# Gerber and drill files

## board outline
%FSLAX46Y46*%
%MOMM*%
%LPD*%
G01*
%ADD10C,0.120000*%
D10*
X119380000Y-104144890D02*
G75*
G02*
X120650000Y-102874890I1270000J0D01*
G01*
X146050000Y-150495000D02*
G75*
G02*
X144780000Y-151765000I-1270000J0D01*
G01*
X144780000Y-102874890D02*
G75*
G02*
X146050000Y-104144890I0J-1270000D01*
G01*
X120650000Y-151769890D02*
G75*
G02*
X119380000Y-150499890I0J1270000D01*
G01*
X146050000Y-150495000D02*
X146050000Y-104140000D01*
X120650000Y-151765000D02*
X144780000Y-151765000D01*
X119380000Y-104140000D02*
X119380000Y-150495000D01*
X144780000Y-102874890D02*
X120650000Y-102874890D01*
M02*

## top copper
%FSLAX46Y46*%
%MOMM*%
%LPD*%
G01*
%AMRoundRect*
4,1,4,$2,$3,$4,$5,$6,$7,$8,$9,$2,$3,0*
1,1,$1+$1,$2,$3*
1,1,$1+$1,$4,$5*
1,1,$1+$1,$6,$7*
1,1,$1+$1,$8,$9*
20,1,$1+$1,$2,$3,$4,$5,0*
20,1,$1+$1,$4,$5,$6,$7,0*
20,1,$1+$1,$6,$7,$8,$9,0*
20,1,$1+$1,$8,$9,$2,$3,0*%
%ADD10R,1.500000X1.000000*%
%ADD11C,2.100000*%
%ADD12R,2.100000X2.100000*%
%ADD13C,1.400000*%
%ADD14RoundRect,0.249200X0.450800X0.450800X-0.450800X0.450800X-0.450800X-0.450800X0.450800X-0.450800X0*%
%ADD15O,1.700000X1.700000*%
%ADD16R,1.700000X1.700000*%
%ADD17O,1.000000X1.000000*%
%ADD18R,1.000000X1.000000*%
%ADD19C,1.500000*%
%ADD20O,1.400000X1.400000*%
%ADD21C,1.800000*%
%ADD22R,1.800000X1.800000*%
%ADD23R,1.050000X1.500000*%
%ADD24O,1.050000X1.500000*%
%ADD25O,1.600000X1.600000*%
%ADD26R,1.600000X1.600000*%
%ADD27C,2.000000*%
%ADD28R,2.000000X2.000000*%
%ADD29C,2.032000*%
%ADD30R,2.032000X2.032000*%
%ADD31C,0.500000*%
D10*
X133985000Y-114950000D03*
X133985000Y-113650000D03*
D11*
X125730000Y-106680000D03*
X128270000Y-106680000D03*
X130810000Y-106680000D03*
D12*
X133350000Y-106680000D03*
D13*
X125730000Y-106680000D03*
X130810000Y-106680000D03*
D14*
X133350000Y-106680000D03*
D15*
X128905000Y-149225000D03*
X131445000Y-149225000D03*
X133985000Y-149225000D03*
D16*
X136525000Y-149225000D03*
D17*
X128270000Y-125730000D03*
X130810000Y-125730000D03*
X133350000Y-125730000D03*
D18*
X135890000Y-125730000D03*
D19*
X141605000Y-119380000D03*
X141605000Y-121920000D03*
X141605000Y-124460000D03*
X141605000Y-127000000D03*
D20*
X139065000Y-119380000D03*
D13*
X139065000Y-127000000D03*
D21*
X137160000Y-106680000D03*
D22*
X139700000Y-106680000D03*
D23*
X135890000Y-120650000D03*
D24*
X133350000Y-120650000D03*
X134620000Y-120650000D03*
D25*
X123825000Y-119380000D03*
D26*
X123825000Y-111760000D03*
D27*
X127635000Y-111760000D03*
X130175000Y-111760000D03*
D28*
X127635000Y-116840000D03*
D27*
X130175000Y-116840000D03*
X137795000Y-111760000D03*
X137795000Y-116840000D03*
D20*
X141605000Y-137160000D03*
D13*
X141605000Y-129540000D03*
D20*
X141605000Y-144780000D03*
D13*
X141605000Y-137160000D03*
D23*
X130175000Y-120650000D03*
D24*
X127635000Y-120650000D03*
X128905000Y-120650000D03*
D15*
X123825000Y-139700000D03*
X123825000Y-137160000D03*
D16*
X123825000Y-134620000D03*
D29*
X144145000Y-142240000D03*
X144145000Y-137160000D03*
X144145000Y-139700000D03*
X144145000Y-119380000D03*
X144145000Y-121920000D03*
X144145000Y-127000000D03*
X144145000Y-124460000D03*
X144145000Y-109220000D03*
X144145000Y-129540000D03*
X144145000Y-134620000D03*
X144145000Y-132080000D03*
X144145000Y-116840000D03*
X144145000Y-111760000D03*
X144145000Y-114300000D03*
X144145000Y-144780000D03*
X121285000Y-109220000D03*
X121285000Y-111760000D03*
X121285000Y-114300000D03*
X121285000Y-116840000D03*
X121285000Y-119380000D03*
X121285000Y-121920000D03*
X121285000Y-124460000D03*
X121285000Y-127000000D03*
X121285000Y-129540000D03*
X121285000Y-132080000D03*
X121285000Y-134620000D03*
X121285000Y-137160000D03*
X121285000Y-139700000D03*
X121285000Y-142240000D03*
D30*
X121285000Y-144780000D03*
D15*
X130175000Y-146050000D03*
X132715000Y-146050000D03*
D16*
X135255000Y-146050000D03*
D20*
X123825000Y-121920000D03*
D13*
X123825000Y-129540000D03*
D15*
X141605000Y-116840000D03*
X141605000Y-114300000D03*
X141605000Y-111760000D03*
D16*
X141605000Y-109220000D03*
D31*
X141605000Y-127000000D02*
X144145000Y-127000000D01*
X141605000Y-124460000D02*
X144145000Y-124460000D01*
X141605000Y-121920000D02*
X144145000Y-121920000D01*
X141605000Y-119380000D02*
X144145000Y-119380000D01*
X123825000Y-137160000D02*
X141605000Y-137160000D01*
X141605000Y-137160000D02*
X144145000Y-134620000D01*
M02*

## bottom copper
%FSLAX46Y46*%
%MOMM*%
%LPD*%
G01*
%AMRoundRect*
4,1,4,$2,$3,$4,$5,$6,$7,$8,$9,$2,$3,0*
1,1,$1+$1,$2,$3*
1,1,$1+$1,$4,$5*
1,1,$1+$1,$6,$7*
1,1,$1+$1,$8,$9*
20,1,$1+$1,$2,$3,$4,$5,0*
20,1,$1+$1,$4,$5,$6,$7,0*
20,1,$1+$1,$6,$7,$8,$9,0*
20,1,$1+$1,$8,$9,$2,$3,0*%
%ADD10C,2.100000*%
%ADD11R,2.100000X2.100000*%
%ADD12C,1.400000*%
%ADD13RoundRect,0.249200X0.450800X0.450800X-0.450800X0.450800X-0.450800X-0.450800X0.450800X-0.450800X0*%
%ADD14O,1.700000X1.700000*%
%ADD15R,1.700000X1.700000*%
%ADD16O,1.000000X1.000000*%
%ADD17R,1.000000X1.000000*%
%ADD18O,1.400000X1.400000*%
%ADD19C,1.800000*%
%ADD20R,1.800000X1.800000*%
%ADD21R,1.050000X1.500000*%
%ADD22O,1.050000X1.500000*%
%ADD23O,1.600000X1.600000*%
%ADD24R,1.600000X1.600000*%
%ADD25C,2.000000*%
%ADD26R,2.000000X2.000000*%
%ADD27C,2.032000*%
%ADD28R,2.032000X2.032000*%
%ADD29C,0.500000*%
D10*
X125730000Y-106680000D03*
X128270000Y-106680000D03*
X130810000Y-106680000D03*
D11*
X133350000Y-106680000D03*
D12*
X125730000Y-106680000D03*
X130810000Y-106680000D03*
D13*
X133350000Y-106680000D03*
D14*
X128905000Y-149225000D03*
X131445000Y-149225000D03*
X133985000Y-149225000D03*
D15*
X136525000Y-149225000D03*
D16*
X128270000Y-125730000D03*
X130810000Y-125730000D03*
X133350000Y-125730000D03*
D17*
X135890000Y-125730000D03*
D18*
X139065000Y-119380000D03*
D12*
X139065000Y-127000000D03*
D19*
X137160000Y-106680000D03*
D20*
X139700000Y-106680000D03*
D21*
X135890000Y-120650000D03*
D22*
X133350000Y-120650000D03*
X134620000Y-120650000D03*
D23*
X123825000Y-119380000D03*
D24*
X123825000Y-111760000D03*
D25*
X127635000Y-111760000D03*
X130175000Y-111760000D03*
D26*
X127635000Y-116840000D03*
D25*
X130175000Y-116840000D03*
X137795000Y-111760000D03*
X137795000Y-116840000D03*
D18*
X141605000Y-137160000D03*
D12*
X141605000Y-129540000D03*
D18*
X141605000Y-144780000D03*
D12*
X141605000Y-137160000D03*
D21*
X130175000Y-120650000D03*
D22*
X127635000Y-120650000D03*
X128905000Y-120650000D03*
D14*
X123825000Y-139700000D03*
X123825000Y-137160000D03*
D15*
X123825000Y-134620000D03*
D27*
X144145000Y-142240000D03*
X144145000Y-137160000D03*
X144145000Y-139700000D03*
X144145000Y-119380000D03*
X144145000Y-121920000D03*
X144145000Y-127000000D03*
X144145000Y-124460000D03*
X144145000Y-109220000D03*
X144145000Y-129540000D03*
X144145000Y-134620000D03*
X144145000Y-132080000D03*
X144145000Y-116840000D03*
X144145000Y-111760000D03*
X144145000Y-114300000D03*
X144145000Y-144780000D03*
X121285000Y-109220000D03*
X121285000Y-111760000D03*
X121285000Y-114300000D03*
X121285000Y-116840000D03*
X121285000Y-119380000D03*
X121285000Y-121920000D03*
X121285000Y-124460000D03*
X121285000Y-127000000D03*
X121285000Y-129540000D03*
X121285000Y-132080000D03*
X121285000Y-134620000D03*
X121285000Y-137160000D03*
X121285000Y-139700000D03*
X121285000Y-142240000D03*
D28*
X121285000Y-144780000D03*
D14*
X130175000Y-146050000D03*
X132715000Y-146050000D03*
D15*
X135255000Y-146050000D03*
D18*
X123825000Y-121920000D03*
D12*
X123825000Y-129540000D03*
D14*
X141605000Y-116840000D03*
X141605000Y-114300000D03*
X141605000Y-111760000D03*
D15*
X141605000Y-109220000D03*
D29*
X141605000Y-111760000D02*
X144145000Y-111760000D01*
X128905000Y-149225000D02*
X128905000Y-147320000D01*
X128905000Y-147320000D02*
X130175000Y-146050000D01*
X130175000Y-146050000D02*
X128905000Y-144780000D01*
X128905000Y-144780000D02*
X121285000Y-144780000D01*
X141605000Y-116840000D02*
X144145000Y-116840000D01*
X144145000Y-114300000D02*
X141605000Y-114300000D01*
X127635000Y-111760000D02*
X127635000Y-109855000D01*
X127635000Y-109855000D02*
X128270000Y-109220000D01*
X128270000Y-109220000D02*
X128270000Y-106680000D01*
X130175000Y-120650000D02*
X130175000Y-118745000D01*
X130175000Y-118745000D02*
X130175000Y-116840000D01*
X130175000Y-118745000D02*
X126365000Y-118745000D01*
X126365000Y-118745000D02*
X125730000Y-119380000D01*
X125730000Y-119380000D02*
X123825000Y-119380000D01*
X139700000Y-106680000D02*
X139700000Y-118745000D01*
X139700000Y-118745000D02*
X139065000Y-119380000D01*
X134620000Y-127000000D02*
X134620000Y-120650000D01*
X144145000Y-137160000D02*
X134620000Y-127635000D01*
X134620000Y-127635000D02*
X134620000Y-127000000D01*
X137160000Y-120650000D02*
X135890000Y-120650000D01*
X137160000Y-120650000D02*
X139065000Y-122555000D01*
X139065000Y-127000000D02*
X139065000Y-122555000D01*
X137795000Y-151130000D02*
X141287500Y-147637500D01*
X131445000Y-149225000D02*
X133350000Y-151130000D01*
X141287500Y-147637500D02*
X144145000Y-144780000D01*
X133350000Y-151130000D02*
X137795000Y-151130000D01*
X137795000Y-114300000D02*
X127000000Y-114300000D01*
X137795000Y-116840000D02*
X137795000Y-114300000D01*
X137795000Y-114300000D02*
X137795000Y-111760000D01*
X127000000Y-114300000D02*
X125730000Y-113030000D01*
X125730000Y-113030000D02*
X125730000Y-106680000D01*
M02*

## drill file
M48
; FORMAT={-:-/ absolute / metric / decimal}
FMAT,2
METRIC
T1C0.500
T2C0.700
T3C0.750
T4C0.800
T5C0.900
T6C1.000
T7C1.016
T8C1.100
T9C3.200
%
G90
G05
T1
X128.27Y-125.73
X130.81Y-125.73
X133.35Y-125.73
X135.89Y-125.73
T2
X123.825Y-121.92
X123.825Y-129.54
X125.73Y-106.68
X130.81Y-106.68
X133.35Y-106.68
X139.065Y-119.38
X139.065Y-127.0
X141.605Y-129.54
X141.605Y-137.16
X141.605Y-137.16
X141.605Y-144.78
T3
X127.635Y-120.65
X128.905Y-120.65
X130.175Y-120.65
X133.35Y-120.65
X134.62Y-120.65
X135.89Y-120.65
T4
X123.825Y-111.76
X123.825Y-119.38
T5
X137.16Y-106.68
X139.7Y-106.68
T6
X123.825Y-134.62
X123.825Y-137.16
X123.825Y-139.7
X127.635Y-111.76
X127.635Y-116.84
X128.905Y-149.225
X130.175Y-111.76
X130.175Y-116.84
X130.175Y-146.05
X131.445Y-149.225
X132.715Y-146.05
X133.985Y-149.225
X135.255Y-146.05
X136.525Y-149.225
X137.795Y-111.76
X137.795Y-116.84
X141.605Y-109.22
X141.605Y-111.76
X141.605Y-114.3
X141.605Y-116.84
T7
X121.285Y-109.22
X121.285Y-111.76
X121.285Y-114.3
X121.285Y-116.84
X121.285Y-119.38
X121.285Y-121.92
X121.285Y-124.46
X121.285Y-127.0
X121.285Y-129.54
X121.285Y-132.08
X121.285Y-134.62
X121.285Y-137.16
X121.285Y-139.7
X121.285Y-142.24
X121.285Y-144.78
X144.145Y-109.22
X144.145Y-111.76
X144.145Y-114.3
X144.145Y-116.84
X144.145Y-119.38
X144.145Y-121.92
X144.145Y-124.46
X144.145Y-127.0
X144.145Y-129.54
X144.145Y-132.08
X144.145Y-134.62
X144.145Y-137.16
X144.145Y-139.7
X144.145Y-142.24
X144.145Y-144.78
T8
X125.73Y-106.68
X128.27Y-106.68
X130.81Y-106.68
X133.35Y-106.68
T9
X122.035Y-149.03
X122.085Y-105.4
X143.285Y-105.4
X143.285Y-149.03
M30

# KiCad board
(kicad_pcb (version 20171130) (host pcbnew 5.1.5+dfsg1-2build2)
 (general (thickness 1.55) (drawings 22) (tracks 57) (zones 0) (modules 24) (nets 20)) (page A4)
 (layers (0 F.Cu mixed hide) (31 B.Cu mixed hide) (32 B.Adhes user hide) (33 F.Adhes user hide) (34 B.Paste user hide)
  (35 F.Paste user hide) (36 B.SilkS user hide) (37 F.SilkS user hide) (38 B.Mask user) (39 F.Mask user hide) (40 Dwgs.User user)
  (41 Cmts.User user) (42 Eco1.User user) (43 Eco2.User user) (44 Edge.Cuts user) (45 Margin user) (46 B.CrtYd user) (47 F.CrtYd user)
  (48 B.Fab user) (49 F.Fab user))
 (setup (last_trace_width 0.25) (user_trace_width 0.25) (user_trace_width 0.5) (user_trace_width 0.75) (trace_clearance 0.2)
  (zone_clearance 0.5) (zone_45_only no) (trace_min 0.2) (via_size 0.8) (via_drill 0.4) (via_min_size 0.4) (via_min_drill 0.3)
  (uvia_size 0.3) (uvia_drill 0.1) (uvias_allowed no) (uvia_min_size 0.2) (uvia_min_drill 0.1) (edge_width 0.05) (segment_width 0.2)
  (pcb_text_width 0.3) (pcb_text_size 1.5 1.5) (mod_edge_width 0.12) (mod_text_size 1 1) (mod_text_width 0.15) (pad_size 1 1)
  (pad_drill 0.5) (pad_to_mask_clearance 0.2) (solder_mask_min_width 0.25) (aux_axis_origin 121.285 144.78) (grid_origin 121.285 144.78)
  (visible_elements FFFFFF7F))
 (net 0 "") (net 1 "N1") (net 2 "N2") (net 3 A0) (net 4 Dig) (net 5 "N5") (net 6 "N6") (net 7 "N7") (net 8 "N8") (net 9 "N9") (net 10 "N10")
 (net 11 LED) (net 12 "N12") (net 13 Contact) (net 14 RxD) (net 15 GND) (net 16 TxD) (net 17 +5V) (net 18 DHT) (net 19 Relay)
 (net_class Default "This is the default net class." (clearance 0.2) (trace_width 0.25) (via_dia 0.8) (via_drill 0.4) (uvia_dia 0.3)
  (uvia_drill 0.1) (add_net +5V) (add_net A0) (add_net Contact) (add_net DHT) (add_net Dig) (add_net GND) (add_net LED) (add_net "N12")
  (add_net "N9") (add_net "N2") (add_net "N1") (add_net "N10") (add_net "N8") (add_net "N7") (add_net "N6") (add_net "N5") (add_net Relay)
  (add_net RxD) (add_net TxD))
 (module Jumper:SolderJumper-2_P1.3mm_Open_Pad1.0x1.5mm (layer F.Cu) (at 133.985 114.3 90)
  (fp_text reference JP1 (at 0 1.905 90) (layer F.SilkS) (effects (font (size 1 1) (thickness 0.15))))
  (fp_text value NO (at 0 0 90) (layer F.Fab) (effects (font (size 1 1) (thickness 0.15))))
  (pad 1 smd rect (at -0.65 0 90) (size 1 1.5) (layers F.Cu F.Mask))
  (pad 2 smd rect (at 0.65 0 90) (size 1 1.5) (layers F.Cu F.Mask)))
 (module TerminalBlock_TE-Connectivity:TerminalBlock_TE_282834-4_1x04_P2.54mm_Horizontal (layer F.Cu) (at 133.35 106.68 180)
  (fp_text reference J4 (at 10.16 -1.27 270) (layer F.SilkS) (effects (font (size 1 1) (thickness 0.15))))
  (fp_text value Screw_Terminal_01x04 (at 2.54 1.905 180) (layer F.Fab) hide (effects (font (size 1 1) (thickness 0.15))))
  (pad 4 thru_hole circle (at 7.62 0 180) (size 2.1 2.1) (drill 1.1) (layers *.Cu *.Mask) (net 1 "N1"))
  (pad 3 thru_hole circle (at 5.08 0 180) (size 2.1 2.1) (drill 1.1) (layers *.Cu *.Mask) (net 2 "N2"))
  (pad 2 thru_hole circle (at 2.54 0 180) (size 2.1 2.1) (drill 1.1) (layers *.Cu *.Mask))
  (pad 1 thru_hole rect (at 0 0 180) (size 2.1 2.1) (drill 1.1) (layers *.Cu *.Mask)))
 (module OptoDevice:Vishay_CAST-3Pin (layer F.Cu) (at 133.35 106.68 180)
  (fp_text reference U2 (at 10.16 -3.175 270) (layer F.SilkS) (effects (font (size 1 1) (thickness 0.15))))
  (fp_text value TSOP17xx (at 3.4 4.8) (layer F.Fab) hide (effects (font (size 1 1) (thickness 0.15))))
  (pad 3 thru_hole circle (at 7.62 0 180) (size 1.4 1.4) (drill 0.7) (layers *.Cu *.Mask) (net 1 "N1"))
  (pad 2 thru_hole circle (at 2.54 0 180) (size 1.4 1.4) (drill 0.7) (layers *.Cu *.Mask))
  (pad 1 thru_hole roundrect (at 0 0 180) (size 1.4 1.4) (drill 0.7) (layers *.Cu *.Mask) (roundrect_rratio 0.178)))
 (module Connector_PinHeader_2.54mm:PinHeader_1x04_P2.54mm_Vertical (layer F.Cu) (at 136.525 149.225 270)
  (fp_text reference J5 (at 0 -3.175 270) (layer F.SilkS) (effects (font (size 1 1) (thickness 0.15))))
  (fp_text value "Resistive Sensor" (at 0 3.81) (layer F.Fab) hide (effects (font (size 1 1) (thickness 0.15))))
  (pad 4 thru_hole oval (at 0 7.62 270) (size 1.7 1.7) (drill 1) (layers *.Cu *.Mask) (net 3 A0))
  (pad 3 thru_hole oval (at 0 5.08 270) (size 1.7 1.7) (drill 1) (layers *.Cu *.Mask) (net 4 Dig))
  (pad 2 thru_hole oval (at 0 2.54 270) (size 1.7 1.7) (drill 1) (layers *.Cu *.Mask))
  (pad 1 thru_hole rect (at 0 0 270) (size 1.7 1.7) (drill 1) (layers *.Cu *.Mask)))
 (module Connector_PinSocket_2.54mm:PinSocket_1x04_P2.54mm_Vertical (layer F.Cu) (at 135.89 125.73 270)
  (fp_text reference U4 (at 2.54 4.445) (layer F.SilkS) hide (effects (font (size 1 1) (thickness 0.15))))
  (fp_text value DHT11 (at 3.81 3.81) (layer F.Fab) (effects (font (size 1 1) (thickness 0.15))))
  (pad 4 thru_hole oval (at 0 7.62 270) (size 1 1) (drill 0.5) (layers *.Cu *.Mask))
  (pad 3 thru_hole oval (at 0 5.08 270) (size 1 1) (drill 0.5) (layers *.Cu *.Mask))
  (pad 2 thru_hole oval (at 0 2.54 270) (size 1 1) (drill 0.5) (layers *.Cu *.Mask))
  (pad 1 thru_hole rect (at 0 0 270) (size 1 1) (drill 0.5) (layers *.Cu *.Mask)))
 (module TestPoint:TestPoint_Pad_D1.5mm (layer F.Cu) (at 141.605 119.38)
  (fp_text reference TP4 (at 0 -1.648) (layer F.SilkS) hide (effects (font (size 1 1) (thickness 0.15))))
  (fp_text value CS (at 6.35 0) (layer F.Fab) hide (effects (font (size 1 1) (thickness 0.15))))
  (pad 1 smd circle (at 0 0) (size 1.5 1.5) (layers F.Cu F.Mask) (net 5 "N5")))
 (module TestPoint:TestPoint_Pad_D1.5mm (layer F.Cu) (at 141.605 121.92)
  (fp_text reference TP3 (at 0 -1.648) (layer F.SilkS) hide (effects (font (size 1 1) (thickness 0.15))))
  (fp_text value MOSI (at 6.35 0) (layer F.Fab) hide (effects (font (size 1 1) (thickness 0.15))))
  (pad 1 smd circle (at 0 0) (size 1.5 1.5) (layers F.Cu F.Mask) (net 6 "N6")))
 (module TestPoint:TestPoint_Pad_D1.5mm (layer F.Cu) (at 141.605 124.46)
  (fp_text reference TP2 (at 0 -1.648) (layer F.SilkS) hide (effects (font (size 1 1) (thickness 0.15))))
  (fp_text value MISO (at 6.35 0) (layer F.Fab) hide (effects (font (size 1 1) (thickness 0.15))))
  (pad 1 smd circle (at 0 0) (size 1.5 1.5) (layers F.Cu F.Mask) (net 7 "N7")))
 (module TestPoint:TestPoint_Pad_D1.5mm (layer F.Cu) (at 141.605 127)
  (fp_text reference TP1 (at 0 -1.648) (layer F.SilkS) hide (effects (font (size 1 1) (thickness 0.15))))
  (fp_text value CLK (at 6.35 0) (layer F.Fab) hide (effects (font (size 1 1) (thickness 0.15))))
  (pad 1 smd circle (at 0 0) (size 1.5 1.5) (layers F.Cu F.Mask) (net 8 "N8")))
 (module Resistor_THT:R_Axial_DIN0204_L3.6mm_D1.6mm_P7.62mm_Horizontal (layer F.Cu) (at 139.065 127 90)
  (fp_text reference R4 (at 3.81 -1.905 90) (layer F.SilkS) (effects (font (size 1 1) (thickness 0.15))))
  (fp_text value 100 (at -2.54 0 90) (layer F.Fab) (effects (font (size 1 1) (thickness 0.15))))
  (pad 2 thru_hole oval (at 7.62 0 90) (size 1.4 1.4) (drill 0.7) (layers *.Cu *.Mask) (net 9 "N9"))
  (pad 1 thru_hole circle (at 0 0 90) (size 1.4 1.4) (drill 0.7) (layers *.Cu *.Mask) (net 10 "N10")))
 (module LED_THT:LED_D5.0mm (layer F.Cu) (at 139.7 106.68 180)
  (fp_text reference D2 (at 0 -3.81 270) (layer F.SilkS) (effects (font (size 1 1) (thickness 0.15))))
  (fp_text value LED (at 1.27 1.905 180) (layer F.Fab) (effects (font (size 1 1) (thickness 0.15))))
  (pad 2 thru_hole circle (at 2.54 0 180) (size 1.8 1.8) (drill 0.9) (layers *.Cu *.Mask))
  (pad 1 thru_hole rect (at 0 0 180) (size 1.8 1.8) (drill 0.9) (layers *.Cu *.Mask) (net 9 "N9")))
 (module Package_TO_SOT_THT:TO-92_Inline (layer F.Cu) (at 135.89 120.65 180)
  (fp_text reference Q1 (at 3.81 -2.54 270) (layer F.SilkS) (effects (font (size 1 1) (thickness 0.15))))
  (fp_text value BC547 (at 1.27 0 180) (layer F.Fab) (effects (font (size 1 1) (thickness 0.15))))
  (pad 1 thru_hole rect (at 0 0 180) (size 1.05 1.5) (drill 0.75) (layers *.Cu *.Mask) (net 10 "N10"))
  (pad 3 thru_hole oval (at 2.54 0 180) (size 1.05 1.5) (drill 0.75) (layers *.Cu *.Mask))
  (pad 2 thru_hole oval (at 1.27 0 180) (size 1.05 1.5) (drill 0.75) (layers *.Cu *.Mask) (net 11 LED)))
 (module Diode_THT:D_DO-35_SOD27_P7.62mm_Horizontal (layer F.Cu) (at 123.825 111.76 270)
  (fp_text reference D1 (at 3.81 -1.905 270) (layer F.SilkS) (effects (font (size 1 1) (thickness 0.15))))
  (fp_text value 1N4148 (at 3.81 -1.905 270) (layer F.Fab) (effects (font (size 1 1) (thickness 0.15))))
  (pad 2 thru_hole oval (at 7.62 0 270) (size 1.6 1.6) (drill 0.8) (layers *.Cu *.Mask) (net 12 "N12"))
  (pad 1 thru_hole rect (at 0 0 270) (size 1.6 1.6) (drill 0.8) (layers *.Cu *.Mask)))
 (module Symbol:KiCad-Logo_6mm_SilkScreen (layer B.Cu) (at 131.445 135.255 90)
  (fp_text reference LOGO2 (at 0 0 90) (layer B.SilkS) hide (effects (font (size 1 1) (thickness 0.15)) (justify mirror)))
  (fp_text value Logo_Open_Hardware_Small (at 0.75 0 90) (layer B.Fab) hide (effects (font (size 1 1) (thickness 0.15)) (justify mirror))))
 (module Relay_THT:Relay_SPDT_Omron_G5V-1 (layer F.Cu) (at 127.635 116.84 90)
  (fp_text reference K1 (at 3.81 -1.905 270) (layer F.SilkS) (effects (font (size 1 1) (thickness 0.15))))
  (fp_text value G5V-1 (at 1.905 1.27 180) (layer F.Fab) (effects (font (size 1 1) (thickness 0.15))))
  (pad 10 thru_hole circle (at 5.08 0 90) (size 2 2) (drill 1) (layers *.Cu *.Mask) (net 2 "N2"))
  (pad 9 thru_hole circle (at 5.08 2.54 90) (size 2 2) (drill 1) (layers *.Cu *.Mask))
  (pad 1 thru_hole rect (at 0 0 90) (size 2 2) (drill 1) (layers *.Cu *.Mask))
  (pad 2 thru_hole circle (at 0 2.54 90) (size 2 2) (drill 1) (layers *.Cu *.Mask) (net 12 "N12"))
  (pad 6 thru_hole circle (at 5.08 10.16 90) (size 2 2) (drill 1) (layers *.Cu *.Mask) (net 1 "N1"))
  (pad 5 thru_hole circle (at 0 10.16 90) (size 2 2) (drill 1) (layers *.Cu *.Mask) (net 1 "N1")))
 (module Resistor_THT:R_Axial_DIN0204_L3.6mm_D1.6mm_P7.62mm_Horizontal (layer F.Cu) (at 141.605 129.54 270)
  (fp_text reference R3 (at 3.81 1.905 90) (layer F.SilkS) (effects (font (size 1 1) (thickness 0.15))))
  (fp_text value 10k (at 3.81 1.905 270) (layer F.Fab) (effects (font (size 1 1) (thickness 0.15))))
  (pad 2 thru_hole oval (at 7.62 0 270) (size 1.4 1.4) (drill 0.7) (layers *.Cu *.Mask) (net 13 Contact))
  (pad 1 thru_hole circle (at 0 0 270) (size 1.4 1.4) (drill 0.7) (layers *.Cu *.Mask)))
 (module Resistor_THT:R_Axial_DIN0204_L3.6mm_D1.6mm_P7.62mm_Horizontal (layer F.Cu) (at 141.605 137.16 270)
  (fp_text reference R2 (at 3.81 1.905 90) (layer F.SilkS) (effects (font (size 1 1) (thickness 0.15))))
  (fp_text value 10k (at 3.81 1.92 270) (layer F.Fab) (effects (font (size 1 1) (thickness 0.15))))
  (pad 2 thru_hole oval (at 7.62 0 270) (size 1.4 1.4) (drill 0.7) (layers *.Cu *.Mask))
  (pad 1 thru_hole circle (at 0 0 270) (size 1.4 1.4) (drill 0.7) (layers *.Cu *.Mask) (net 13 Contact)))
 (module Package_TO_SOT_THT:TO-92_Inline (layer F.Cu) (at 130.175 120.65 180)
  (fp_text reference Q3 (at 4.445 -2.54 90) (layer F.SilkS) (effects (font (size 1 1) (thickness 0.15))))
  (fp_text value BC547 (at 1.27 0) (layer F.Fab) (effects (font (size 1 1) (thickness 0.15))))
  (pad 1 thru_hole rect (at 0 0 180) (size 1.05 1.5) (drill 0.75) (layers *.Cu *.Mask) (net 12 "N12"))
  (pad 3 thru_hole oval (at 2.54 0 180) (size 1.05 1.5) (drill 0.75) (layers *.Cu *.Mask))
  (pad 2 thru_hole oval (at 1.27 0 180) (size 1.05 1.5) (drill 0.75) (layers *.Cu *.Mask)))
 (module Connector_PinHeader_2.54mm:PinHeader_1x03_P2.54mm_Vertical (layer F.Cu) (at 123.825 134.62)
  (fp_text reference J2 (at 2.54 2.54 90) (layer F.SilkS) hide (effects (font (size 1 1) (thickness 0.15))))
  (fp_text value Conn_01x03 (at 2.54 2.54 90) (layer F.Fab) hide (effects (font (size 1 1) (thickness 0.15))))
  (pad 3 thru_hole oval (at 0 5.08) (size 1.7 1.7) (drill 1) (layers *.Cu *.Mask))
  (pad 2 thru_hole oval (at 0 2.54) (size 1.7 1.7) (drill 1) (layers *.Cu *.Mask) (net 13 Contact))
  (pad 1 thru_hole rect (at 0 0) (size 1.7 1.7) (drill 1) (layers *.Cu *.Mask)))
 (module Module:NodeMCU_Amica (layer B.Cu) (at 121.285 144.78)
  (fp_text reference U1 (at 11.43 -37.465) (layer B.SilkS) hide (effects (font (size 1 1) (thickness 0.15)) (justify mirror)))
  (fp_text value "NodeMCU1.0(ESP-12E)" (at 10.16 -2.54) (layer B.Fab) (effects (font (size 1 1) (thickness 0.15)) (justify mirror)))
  (pad "" np_thru_hole circle (at 0.75 4.25) (size 3.2 3.2) (drill 3.2) (layers *.Cu *.Mask))
  (pad "" np_thru_hole circle (at 22 4.25) (size 3.2 3.2) (drill 3.2) (layers *.Cu *.Mask))
  (pad "" np_thru_hole circle (at 22 -39.38) (size 3.2 3.2) (drill 3.2) (layers *.Cu *.Mask))
  (pad "" np_thru_hole circle (at 0.8 -39.38) (size 3.2 3.2) (drill 3.2) (layers *.Cu *.Mask))
  (pad 29 thru_hole circle (at 22.86 -2.54) (size 2.032 2.032) (drill 1.016) (layers *.Cu *.Mask))
  (pad 27 thru_hole circle (at 22.86 -7.62) (size 2.032 2.032) (drill 1.016) (layers *.Cu *.Mask) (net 11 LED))
  (pad 28 thru_hole circle (at 22.86 -5.08) (size 2.032 2.032) (drill 1.016) (layers *.Cu *.Mask))
  (pad 20 thru_hole circle (at 22.86 -25.4) (size 2.032 2.032) (drill 1.016) (layers *.Cu *.Mask) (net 5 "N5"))
  (pad 21 thru_hole circle (at 22.86 -22.86) (size 2.032 2.032) (drill 1.016) (layers *.Cu *.Mask) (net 6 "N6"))
  (pad 23 thru_hole circle (at 22.86 -17.78) (size 2.032 2.032) (drill 1.016) (layers *.Cu *.Mask) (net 8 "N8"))
  (pad 22 thru_hole circle (at 22.86 -20.32) (size 2.032 2.032) (drill 1.016) (layers *.Cu *.Mask) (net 7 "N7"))
  (pad 16 thru_hole circle (at 22.86 -35.56) (size 2.032 2.032) (drill 1.016) (layers *.Cu *.Mask))
  (pad 24 thru_hole circle (at 22.86 -15.24) (size 2.032 2.032) (drill 1.016) (layers *.Cu *.Mask))
  (pad 26 thru_hole circle (at 22.86 -10.16) (size 2.032 2.032) (drill 1.016) (layers *.Cu *.Mask) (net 13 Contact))
  (pad 25 thru_hole circle (at 22.86 -12.7) (size 2.032 2.032) (drill 1.016) (layers *.Cu *.Mask))
  (pad 19 thru_hole circle (at 22.86 -27.94) (size 2.032 2.032) (drill 1.016) (layers *.Cu *.Mask) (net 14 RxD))
  (pad 17 thru_hole circle (at 22.86 -33.02) (size 2.032 2.032) (drill 1.016) (layers *.Cu *.Mask) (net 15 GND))
  (pad 18 thru_hole circle (at 22.86 -30.48) (size 2.032 2.032) (drill 1.016) (layers *.Cu *.Mask) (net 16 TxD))
  (pad 30 thru_hole circle (at 22.86 0) (size 2.032 2.032) (drill 1.016) (layers *.Cu *.Mask) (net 4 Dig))
  (pad 15 thru_hole circle (at 0 -35.56) (size 2.032 2.032) (drill 1.016) (layers *.Cu *.Mask))
  (pad 14 thru_hole circle (at 0 -33.02) (size 2.032 2.032) (drill 1.016) (layers *.Cu *.Mask))
  (pad 13 thru_hole circle (at 0 -30.48) (size 2.032 2.032) (drill 1.016) (layers *.Cu *.Mask))
  (pad 12 thru_hole circle (at 0 -27.94) (size 2.032 2.032) (drill 1.016) (layers *.Cu *.Mask))
  (pad 11 thru_hole circle (at 0 -25.4) (size 2.032 2.032) (drill 1.016) (layers *.Cu *.Mask))
  (pad 10 thru_hole circle (at 0 -22.86) (size 2.032 2.032) (drill 1.016) (layers *.Cu *.Mask))
  (pad 9 thru_hole circle (at 0 -20.32) (size 2.032 2.032) (drill 1.016) (layers *.Cu *.Mask))
  (pad 8 thru_hole circle (at 0 -17.78) (size 2.032 2.032) (drill 1.016) (layers *.Cu *.Mask))
  (pad 7 thru_hole circle (at 0 -15.24) (size 2.032 2.032) (drill 1.016) (layers *.Cu *.Mask))
  (pad 6 thru_hole circle (at 0 -12.7) (size 2.032 2.032) (drill 1.016) (layers *.Cu *.Mask))
  (pad 5 thru_hole circle (at 0 -10.16) (size 2.032 2.032) (drill 1.016) (layers *.Cu *.Mask))
  (pad 4 thru_hole circle (at 0 -7.62) (size 2.032 2.032) (drill 1.016) (layers *.Cu *.Mask))
  (pad 3 thru_hole circle (at 0 -5.08) (size 2.032 2.032) (drill 1.016) (layers *.Cu *.Mask))
  (pad 2 thru_hole circle (at 0 -2.54) (size 2.032 2.032) (drill 1.016) (layers *.Cu *.Mask))
  (pad 1 thru_hole rect (at 0 0) (size 2.032 2.032) (drill 1.016) (layers *.Cu *.Mask) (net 3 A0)))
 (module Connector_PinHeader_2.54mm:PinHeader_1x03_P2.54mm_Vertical (layer F.Cu) (at 135.255 146.05 270)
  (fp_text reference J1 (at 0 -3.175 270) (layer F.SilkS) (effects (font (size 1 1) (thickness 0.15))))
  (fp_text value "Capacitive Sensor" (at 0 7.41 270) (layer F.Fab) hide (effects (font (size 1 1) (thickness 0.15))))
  (pad 3 thru_hole oval (at 0 5.08 270) (size 1.7 1.7) (drill 1) (layers *.Cu *.Mask) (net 3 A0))
  (pad 2 thru_hole oval (at 0 2.54 270) (size 1.7 1.7) (drill 1) (layers *.Cu *.Mask))
  (pad 1 thru_hole rect (at 0 0 270) (size 1.7 1.7) (drill 1) (layers *.Cu *.Mask)))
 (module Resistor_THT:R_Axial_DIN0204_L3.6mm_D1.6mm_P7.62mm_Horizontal (layer F.Cu) (at 123.825 129.54 90)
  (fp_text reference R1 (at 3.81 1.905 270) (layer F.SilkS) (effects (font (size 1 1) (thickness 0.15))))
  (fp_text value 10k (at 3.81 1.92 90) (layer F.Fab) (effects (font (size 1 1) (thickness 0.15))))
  (pad 2 thru_hole oval (at 7.62 0 90) (size 1.4 1.4) (drill 0.7) (layers *.Cu *.Mask))
  (pad 1 thru_hole circle (at 0 0 90) (size 1.4 1.4) (drill 0.7) (layers *.Cu *.Mask)))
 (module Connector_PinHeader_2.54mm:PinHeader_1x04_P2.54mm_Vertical (layer F.Cu) (at 141.605 109.22)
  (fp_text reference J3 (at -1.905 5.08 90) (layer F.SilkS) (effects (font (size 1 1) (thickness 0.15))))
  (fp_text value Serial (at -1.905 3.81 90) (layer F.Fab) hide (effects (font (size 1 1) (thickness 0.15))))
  (pad 4 thru_hole oval (at 0 7.62) (size 1.7 1.7) (drill 1) (layers *.Cu *.Mask) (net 14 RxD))
  (pad 3 thru_hole oval (at 0 5.08) (size 1.7 1.7) (drill 1) (layers *.Cu *.Mask) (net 16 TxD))
  (pad 2 thru_hole oval (at 0 2.54) (size 1.7 1.7) (drill 1) (layers *.Cu *.Mask) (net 15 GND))
  (pad 1 thru_hole rect (at 0 0) (size 1.7 1.7) (drill 1) (layers *.Cu *.Mask)))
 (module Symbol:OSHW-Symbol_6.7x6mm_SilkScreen (layer B.Cu) (at 137.795 142.24 90)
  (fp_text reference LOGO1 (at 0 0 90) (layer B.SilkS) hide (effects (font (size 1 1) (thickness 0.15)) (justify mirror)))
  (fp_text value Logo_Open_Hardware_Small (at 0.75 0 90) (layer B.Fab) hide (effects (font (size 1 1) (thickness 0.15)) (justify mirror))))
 (gr_arc (start 120.65 104.14489) (end 120.65 102.87489) (angle -90) (layer Edge.Cuts) (width 0.12))
 (gr_arc (start 144.78 150.495) (end 144.78 151.765) (angle -90) (layer Edge.Cuts) (width 0.12))
 (gr_arc (start 144.78 104.14489) (end 146.05 104.14489) (angle -90) (layer Edge.Cuts) (width 0.12))
 (gr_arc (start 120.65 150.49989) (end 119.38 150.49989) (angle -90) (layer Edge.Cuts) (width 0.12))
 (gr_line (start 146.05 150.495) (end 146.05 104.14) (layer Edge.Cuts) (width 0.12))
 (gr_line (start 120.65 151.765) (end 144.78 151.765) (layer Edge.Cuts) (width 0.12))
 (gr_line (start 119.38 104.14) (end 119.38 150.495) (layer Edge.Cuts) (width 0.12))
 (gr_line (start 144.78 102.87489) (end 120.65 102.87489) (layer Edge.Cuts) (width 0.12))
 (segment (start 141.605 111.76) (end 144.145 111.76) (width 0.5) (layer B.Cu) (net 15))
 (segment (start 128.905 149.225) (end 128.905 147.32) (width 0.5) (layer B.Cu) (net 3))
 (segment (start 128.905 147.32) (end 130.175 146.05) (width 0.5) (layer B.Cu) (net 3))
 (segment (start 130.175 146.05) (end 128.905 144.78) (width 0.5) (layer B.Cu) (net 3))
 (segment (start 128.905 144.78) (end 121.285 144.78) (width 0.5) (layer B.Cu) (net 3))
 (segment (start 141.605 116.84) (end 144.145 116.84) (width 0.5) (layer B.Cu) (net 14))
 (segment (start 144.145 114.3) (end 141.605 114.3) (width 0.5) (layer B.Cu) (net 16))
 (segment (start 127.635 111.76) (end 127.635 109.855) (width 0.5) (layer B.Cu) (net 2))
 (segment (start 127.635 109.855) (end 128.27 109.22) (width 0.5) (layer B.Cu) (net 2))
 (segment (start 128.27 109.22) (end 128.27 106.68) (width 0.5) (layer B.Cu) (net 2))
 (segment (start 130.175 120.65) (end 130.175 118.745) (width 0.5) (layer B.Cu) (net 12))
 (segment (start 130.175 118.745) (end 130.175 116.84) (width 0.5) (layer B.Cu) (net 12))
 (segment (start 130.175 118.745) (end 126.365 118.745) (width 0.5) (layer B.Cu) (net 12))
 (segment (start 126.365 118.745) (end 125.73 119.38) (width 0.5) (layer B.Cu) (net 12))
 (segment (start 125.73 119.38) (end 123.825 119.38) (width 0.5) (layer B.Cu) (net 12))
 (segment (start 139.7 106.68) (end 139.7 118.745) (width 0.5) (layer B.Cu) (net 9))
 (segment (start 139.7 118.745) (end 139.065 119.38) (width 0.5) (layer B.Cu) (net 9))
 (segment (start 134.62 127) (end 134.62 120.65) (width 0.5) (layer B.Cu) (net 11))
 (segment (start 144.145 137.16) (end 134.62 127.635) (width 0.5) (layer B.Cu) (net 11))
 (segment (start 134.62 127.635) (end 134.62 127) (width 0.5) (layer B.Cu) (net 11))
 (segment (start 137.16 120.65) (end 135.89 120.65) (width 0.5) (layer B.Cu) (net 10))
 (segment (start 137.16 120.65) (end 139.065 122.555) (width 0.5) (layer B.Cu) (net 10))
 (segment (start 139.065 127) (end 139.065 122.555) (width 0.5) (layer B.Cu) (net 10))
 (segment (start 141.605 127) (end 144.145 127) (width 0.5) (layer F.Cu) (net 8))
 (segment (start 141.605 124.46) (end 144.145 124.46) (width 0.5) (layer F.Cu) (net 7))
 (segment (start 141.605 121.92) (end 144.145 121.92) (width 0.5) (layer F.Cu) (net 6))
 (segment (start 141.605 119.38) (end 144.145 119.38) (width 0.5) (layer F.Cu) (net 5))
 (segment (start 137.795 151.13) (end 141.2875 147.6375) (width 0.5) (layer B.Cu) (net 4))
 (segment (start 131.445 149.225) (end 133.35 151.13) (width 0.5) (layer B.Cu) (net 4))
 (segment (start 141.2875 147.6375) (end 144.145 144.78) (width 0.5) (layer B.Cu) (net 4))
 (segment (start 133.35 151.13) (end 137.795 151.13) (width 0.5) (layer B.Cu) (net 4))
 (segment (start 123.825 137.16) (end 141.605 137.16) (width 0.5) (layer F.Cu) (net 13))
 (segment (start 141.605 137.16) (end 144.145 134.62) (width 0.5) (layer F.Cu) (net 13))
 (segment (start 137.795 114.3) (end 127 114.3) (width 0.5) (layer B.Cu) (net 1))
 (segment (start 137.795 116.84) (end 137.795 114.3) (width 0.5) (layer B.Cu) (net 1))
 (segment (start 137.795 114.3) (end 137.795 111.76) (width 0.5) (layer B.Cu) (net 1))
 (segment (start 127 114.3) (end 125.73 113.03) (width 0.5) (layer B.Cu) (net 1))
 (segment (start 125.73 113.03) (end 125.73 106.68) (width 0.5) (layer B.Cu) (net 1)))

